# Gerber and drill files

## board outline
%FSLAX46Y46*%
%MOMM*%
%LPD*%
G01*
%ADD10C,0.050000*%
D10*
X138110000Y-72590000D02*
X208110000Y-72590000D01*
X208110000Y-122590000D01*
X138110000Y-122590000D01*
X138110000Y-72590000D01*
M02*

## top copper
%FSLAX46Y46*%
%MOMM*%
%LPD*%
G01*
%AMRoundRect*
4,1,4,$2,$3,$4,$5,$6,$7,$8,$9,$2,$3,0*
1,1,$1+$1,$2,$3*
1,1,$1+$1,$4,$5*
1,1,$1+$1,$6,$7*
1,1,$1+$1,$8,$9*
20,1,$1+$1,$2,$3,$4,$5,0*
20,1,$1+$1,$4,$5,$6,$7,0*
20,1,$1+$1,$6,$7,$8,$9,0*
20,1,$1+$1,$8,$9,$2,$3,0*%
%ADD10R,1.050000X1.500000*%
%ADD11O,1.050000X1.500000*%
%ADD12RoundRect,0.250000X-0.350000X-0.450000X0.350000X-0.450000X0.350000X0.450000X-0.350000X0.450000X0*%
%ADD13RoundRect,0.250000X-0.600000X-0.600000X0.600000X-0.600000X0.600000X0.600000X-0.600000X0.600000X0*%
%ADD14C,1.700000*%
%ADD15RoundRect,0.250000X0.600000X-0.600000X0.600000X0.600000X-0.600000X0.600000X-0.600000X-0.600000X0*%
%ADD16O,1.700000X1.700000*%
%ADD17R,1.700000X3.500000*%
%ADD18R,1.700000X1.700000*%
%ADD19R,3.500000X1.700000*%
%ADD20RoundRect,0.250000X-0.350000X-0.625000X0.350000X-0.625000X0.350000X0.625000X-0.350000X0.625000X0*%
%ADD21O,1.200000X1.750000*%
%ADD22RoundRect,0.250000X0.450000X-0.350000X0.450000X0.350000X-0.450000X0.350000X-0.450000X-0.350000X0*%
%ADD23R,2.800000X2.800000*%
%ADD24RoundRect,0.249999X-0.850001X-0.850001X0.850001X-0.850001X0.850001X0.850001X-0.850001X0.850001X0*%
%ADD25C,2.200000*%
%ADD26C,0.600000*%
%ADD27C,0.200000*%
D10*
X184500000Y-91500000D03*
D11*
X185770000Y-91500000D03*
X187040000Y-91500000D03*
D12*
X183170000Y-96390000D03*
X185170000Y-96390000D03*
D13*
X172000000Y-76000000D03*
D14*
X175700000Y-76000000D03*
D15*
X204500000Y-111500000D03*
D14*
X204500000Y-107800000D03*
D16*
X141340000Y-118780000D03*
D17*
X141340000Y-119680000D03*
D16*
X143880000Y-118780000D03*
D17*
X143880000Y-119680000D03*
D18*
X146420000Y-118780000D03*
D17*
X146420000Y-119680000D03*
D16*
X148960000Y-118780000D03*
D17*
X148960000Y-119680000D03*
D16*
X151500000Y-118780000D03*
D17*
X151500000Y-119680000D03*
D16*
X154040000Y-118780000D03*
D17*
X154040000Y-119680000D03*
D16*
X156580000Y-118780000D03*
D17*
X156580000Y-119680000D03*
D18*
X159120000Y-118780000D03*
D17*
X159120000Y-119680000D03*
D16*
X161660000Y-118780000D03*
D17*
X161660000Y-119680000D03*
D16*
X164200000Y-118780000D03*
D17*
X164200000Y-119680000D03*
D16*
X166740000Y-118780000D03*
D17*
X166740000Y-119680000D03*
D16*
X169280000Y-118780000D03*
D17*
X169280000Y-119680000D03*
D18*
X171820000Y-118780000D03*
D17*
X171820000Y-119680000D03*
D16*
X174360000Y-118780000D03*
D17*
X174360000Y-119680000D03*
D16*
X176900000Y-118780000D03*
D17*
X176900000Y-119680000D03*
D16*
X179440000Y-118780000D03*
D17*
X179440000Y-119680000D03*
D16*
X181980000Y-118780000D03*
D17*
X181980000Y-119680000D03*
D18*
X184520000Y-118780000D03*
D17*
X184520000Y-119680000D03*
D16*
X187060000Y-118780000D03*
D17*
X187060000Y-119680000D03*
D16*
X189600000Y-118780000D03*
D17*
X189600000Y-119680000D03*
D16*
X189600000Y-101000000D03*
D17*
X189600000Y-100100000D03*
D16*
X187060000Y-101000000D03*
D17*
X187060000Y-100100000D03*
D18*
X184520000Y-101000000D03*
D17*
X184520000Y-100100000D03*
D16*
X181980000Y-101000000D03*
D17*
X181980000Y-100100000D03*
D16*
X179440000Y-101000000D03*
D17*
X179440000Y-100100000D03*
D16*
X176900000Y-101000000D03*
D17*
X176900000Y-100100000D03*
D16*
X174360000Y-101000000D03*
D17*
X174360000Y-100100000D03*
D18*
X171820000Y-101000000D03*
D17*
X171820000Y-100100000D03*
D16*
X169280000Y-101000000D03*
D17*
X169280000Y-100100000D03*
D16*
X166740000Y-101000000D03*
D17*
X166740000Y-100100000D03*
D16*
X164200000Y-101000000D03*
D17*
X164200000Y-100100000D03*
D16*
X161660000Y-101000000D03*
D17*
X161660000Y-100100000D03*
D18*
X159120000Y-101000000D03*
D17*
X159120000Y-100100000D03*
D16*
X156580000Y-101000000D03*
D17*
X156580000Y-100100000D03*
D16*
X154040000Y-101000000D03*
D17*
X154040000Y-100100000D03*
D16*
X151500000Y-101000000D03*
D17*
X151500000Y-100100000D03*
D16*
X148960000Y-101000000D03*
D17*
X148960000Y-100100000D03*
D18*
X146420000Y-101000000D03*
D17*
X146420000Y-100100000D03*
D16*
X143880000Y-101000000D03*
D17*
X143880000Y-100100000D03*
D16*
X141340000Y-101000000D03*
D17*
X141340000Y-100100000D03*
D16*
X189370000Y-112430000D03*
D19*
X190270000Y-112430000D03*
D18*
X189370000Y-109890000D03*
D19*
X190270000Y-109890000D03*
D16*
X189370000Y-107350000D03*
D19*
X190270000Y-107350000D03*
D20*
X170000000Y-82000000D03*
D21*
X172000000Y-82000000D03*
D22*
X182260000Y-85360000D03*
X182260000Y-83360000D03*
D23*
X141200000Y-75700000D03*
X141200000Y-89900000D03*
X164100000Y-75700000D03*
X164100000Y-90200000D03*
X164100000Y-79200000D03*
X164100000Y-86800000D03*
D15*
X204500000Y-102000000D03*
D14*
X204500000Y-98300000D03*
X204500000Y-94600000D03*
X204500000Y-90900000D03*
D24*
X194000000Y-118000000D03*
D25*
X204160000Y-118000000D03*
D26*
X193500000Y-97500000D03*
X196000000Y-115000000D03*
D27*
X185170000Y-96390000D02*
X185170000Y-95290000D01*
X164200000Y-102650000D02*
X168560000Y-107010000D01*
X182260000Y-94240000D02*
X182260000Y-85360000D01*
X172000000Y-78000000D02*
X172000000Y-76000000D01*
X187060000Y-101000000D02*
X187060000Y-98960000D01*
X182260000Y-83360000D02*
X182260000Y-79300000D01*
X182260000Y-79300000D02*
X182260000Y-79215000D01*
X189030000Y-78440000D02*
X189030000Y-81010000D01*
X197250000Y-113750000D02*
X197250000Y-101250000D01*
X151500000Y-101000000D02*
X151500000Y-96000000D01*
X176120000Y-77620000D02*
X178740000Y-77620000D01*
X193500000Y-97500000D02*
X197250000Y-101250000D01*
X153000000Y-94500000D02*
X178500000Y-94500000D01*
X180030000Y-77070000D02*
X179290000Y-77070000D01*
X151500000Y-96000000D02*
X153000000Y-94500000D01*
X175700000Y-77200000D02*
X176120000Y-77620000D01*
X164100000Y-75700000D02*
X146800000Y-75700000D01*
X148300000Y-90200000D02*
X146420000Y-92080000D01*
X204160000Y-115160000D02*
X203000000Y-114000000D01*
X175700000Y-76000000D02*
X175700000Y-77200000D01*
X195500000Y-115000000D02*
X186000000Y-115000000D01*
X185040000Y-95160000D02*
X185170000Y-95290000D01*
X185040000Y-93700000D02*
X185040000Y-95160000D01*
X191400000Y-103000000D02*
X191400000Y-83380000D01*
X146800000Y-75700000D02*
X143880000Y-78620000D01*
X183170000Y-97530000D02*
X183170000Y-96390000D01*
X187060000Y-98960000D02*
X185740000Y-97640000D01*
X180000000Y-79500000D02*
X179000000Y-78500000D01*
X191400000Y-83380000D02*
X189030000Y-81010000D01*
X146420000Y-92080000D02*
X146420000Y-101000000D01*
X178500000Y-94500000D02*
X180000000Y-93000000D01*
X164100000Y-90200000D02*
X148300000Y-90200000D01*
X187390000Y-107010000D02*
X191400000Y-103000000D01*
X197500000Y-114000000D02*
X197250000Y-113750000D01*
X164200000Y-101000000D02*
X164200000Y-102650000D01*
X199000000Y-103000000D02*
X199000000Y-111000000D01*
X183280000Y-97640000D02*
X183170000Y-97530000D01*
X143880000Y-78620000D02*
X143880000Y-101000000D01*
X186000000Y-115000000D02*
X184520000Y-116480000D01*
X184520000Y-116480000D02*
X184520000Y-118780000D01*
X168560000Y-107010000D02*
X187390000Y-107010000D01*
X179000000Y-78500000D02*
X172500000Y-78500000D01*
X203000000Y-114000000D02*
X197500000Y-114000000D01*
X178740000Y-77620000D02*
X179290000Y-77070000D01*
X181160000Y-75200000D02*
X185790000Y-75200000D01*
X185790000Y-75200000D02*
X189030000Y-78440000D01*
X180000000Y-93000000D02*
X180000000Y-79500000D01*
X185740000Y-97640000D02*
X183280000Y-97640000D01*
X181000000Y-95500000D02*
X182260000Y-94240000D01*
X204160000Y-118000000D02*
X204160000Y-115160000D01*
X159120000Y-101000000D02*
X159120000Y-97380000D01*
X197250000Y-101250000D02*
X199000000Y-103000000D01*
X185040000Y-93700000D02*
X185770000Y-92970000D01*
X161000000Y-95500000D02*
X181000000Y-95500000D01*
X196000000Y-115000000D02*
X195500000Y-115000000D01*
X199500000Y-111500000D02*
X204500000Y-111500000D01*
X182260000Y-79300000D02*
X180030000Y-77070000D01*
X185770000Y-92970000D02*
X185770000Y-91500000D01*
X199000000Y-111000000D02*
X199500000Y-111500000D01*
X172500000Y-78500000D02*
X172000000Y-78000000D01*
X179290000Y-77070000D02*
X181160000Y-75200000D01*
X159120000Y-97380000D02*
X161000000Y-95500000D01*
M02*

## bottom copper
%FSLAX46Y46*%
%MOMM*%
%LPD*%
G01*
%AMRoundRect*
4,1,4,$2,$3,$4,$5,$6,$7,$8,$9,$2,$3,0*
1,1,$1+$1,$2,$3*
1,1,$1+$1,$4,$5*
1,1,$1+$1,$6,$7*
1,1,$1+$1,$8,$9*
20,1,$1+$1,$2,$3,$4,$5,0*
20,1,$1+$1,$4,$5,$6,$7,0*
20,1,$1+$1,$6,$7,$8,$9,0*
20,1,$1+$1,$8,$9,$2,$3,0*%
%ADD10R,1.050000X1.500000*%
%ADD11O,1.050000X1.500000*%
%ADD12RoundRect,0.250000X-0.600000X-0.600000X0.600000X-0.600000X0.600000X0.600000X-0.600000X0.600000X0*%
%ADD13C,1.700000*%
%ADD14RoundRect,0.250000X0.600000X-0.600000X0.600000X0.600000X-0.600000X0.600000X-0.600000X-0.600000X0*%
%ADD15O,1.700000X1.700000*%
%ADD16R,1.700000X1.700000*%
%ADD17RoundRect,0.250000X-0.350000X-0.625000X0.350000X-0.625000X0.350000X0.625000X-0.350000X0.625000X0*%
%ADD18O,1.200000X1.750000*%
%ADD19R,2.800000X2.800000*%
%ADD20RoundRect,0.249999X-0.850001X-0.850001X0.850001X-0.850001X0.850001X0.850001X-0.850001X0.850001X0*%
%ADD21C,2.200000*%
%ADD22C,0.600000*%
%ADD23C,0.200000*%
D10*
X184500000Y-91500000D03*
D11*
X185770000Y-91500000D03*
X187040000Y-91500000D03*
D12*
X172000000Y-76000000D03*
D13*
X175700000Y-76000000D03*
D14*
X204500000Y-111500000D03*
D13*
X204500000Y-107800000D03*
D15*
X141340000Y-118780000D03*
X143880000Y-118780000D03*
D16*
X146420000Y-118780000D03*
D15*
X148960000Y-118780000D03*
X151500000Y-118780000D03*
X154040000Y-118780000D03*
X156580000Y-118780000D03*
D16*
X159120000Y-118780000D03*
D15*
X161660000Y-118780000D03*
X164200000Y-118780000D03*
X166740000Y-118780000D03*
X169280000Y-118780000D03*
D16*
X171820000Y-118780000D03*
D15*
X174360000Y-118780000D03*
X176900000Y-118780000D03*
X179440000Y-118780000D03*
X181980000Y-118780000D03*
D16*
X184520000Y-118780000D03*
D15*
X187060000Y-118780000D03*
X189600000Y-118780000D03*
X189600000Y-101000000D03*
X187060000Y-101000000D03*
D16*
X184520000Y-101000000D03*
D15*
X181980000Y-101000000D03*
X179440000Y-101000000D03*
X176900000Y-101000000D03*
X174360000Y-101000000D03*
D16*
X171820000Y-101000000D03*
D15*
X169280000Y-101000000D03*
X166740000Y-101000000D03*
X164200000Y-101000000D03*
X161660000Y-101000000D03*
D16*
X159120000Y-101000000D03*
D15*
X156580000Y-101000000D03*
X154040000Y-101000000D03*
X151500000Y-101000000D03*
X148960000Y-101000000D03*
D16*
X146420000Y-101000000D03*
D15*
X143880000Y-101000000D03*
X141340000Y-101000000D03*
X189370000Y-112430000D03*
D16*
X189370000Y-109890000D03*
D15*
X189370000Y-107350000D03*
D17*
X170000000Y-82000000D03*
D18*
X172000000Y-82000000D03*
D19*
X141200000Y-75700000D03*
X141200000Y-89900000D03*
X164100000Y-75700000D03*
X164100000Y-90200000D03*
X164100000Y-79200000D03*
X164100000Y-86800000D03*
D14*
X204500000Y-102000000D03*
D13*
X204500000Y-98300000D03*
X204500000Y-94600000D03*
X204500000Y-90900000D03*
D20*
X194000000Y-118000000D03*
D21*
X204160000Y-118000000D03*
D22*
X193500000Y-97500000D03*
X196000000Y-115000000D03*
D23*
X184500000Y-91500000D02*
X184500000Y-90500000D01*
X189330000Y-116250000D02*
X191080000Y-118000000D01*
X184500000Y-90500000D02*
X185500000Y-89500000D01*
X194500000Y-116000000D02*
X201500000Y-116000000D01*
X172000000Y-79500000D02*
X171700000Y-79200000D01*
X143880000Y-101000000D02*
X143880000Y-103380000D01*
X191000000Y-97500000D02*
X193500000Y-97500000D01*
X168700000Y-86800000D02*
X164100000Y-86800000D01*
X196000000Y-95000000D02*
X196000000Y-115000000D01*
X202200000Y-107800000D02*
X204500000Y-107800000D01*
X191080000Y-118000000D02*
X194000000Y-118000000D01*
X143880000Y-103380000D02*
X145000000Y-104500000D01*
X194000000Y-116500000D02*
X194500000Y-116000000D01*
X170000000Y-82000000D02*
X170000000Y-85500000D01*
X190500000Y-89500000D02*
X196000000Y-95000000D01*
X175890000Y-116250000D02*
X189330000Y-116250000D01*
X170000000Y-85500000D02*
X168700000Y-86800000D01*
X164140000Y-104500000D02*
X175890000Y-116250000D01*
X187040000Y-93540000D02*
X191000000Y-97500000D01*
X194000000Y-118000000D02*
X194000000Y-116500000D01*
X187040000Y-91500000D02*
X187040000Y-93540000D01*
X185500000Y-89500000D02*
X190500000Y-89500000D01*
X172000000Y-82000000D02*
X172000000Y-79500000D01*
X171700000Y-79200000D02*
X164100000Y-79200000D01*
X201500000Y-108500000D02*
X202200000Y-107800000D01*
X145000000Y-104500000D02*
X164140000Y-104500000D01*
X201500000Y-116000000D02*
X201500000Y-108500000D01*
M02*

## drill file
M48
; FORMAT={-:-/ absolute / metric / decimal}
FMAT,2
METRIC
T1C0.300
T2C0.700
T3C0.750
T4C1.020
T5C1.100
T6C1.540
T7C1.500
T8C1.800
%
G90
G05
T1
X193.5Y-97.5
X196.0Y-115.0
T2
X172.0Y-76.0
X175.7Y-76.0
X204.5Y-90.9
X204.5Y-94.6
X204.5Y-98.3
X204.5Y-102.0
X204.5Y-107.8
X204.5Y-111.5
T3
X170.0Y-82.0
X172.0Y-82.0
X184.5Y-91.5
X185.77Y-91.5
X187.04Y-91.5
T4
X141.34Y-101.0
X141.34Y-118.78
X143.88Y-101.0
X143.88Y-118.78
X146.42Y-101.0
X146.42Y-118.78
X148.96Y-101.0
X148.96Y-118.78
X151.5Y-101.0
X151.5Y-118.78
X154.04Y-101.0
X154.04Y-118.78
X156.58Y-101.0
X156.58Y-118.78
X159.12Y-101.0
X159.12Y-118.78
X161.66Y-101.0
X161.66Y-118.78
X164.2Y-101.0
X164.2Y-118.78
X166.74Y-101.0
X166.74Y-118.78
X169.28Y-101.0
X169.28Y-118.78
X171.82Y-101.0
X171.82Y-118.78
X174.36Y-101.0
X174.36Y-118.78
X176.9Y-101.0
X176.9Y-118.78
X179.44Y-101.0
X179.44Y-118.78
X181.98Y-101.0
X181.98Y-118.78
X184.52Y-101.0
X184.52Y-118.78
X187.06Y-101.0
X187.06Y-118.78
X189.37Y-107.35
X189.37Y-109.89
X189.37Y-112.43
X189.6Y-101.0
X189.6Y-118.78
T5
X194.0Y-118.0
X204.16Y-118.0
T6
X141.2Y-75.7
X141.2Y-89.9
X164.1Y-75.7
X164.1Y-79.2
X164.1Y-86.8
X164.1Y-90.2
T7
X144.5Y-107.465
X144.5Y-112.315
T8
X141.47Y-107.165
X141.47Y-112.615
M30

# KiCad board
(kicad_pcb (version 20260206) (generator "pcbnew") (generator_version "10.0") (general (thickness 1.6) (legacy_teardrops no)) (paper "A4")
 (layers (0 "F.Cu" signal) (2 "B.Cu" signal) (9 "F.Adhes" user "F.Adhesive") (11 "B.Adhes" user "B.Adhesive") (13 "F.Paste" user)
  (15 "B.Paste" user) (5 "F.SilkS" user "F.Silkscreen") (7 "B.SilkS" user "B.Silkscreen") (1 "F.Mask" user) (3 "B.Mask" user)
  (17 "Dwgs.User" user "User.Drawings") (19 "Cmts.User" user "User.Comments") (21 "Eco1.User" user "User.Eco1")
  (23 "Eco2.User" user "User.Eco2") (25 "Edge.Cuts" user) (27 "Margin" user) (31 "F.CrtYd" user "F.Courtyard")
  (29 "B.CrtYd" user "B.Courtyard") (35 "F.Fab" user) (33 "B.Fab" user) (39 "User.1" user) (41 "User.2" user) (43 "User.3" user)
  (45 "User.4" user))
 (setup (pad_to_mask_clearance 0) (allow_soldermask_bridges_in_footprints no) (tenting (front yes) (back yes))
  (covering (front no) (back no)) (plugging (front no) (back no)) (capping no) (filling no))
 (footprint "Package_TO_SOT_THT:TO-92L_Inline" (layer "F.Cu") (at 184.5 91.5)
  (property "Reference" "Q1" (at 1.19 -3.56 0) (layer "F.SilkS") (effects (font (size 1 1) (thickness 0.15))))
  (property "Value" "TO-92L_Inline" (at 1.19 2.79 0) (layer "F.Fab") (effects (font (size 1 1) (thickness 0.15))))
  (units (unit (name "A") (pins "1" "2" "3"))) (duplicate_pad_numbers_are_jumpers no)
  (pad "1" thru_hole rect (at 0 0) (size 1.05 1.5) (drill 0.75) (layers "*.Cu" "*.Mask") (remove_unused_layers no))
  (pad "2" thru_hole oval (at 1.27 0) (size 1.05 1.5) (drill 0.75) (layers "*.Cu" "*.Mask") (remove_unused_layers no))
  (pad "3" thru_hole oval (at 2.54 0) (size 1.05 1.5) (drill 0.75) (layers "*.Cu" "*.Mask") (remove_unused_layers no)))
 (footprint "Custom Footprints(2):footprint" (layer "F.Cu") (at 202 78.55)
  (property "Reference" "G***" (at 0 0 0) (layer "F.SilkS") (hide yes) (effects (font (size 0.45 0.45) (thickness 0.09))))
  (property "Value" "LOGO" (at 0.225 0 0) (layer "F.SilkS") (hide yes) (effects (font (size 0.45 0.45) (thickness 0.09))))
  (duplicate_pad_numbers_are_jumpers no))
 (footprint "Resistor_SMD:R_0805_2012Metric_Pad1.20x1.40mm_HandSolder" (layer "F.Cu") (at 184.17 96.39)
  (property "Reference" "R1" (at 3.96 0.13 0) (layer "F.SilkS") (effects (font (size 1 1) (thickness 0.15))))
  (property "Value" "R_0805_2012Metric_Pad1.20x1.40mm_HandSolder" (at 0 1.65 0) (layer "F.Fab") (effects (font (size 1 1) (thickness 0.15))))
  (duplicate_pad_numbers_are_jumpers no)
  (pad "1" smd roundrect (at -1 0) (size 1.2 1.4) (layers "F.Cu" "F.Mask" "F.Paste") (roundrect_rratio 0.208333))
  (pad "2" smd roundrect (at 1 0) (size 1.2 1.4) (layers "F.Cu" "F.Mask" "F.Paste") (roundrect_rratio 0.208333)))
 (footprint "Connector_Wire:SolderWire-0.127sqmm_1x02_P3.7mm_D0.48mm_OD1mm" (layer "F.Cu") (at 172 76)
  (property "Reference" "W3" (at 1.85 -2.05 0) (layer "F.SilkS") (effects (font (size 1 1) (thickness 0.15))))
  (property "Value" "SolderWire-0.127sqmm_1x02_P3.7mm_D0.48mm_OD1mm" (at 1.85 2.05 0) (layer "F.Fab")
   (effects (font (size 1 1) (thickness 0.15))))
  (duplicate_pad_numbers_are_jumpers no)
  (pad "1" thru_hole roundrect (at 0 0) (size 1.7 1.7) (drill 0.7) (layers "*.Cu" "*.Mask") (remove_unused_layers no)
   (roundrect_rratio 0.147059))
  (pad "2" thru_hole circle (at 3.7 0) (size 1.7 1.7) (drill 0.7) (layers "*.Cu" "*.Mask") (remove_unused_layers no)))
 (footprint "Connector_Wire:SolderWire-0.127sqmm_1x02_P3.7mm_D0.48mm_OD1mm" (layer "F.Cu") (at 204.5 111.5 90)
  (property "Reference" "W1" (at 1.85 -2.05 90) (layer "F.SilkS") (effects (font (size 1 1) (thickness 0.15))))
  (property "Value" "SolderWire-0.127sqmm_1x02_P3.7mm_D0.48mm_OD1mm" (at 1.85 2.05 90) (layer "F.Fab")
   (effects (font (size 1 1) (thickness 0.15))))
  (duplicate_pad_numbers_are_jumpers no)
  (pad "1" thru_hole roundrect (at 0 0 90) (size 1.7 1.7) (drill 0.7) (layers "*.Cu" "*.Mask") (remove_unused_layers no)
   (roundrect_rratio 0.147059))
  (pad "2" thru_hole circle (at 3.7 0 90) (size 1.7 1.7) (drill 0.7) (layers "*.Cu" "*.Mask") (remove_unused_layers no)))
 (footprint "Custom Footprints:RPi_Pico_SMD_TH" (layer "F.Cu") (at 165.47 109.89 90)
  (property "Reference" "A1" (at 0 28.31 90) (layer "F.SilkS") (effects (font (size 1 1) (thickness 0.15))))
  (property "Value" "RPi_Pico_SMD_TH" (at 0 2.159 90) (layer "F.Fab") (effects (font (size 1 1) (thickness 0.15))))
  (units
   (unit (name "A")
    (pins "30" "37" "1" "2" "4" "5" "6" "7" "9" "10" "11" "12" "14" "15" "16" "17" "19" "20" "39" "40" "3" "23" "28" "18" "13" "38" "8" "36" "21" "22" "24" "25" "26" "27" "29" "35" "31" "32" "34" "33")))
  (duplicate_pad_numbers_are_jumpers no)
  (pad "" np_thru_hole oval (at -2.725 -24 90) (size 1.8 1.8) (drill 1.8) (layers "*.Cu" "*.Mask"))
  (pad "" np_thru_hole oval (at -2.425 -20.97 90) (size 1.5 1.5) (drill 1.5) (layers "*.Cu" "*.Mask"))
  (pad "" np_thru_hole oval (at 2.425 -20.97 90) (size 1.5 1.5) (drill 1.5) (layers "*.Cu" "*.Mask"))
  (pad "" np_thru_hole oval (at 2.725 -24 90) (size 1.8 1.8) (drill 1.8) (layers "*.Cu" "*.Mask"))
  (pad "1" thru_hole oval (at -8.89 -24.13 90) (size 1.7 1.7) (drill 1.02) (layers "*.Cu" "*.Mask") (remove_unused_layers no))
  (pad "1" smd rect (at -8.89 -24.13 90) (size 3.5 1.7) (drill (offset -0.9 0)) (layers "F.Cu" "F.Mask"))
  (pad "2" thru_hole oval (at -8.89 -21.59 90) (size 1.7 1.7) (drill 1.02) (layers "*.Cu" "*.Mask") (remove_unused_layers no))
  (pad "2" smd rect (at -8.89 -21.59 90) (size 3.5 1.7) (drill (offset -0.9 0)) (layers "F.Cu" "F.Mask"))
  (pad "3" thru_hole rect (at -8.89 -19.05 90) (size 1.7 1.7) (drill 1.02) (layers "*.Cu" "*.Mask") (remove_unused_layers no))
  (pad "3" smd rect (at -8.89 -19.05 90) (size 3.5 1.7) (drill (offset -0.9 0)) (layers "F.Cu" "F.Mask"))
  (pad "4" thru_hole oval (at -8.89 -16.51 90) (size 1.7 1.7) (drill 1.02) (layers "*.Cu" "*.Mask") (remove_unused_layers no))
  (pad "4" smd rect (at -8.89 -16.51 90) (size 3.5 1.7) (drill (offset -0.9 0)) (layers "F.Cu" "F.Mask"))
  (pad "5" thru_hole oval (at -8.89 -13.97 90) (size 1.7 1.7) (drill 1.02) (layers "*.Cu" "*.Mask") (remove_unused_layers no))
  (pad "5" smd rect (at -8.89 -13.97 90) (size 3.5 1.7) (drill (offset -0.9 0)) (layers "F.Cu" "F.Mask"))
  (pad "6" thru_hole oval (at -8.89 -11.43 90) (size 1.7 1.7) (drill 1.02) (layers "*.Cu" "*.Mask") (remove_unused_layers no))
  (pad "6" smd rect (at -8.89 -11.43 90) (size 3.5 1.7) (drill (offset -0.9 0)) (layers "F.Cu" "F.Mask"))
  (pad "7" thru_hole oval (at -8.89 -8.89 90) (size 1.7 1.7) (drill 1.02) (layers "*.Cu" "*.Mask") (remove_unused_layers no))
  (pad "7" smd rect (at -8.89 -8.89 90) (size 3.5 1.7) (drill (offset -0.9 0)) (layers "F.Cu" "F.Mask"))
  (pad "8" thru_hole rect (at -8.89 -6.35 90) (size 1.7 1.7) (drill 1.02) (layers "*.Cu" "*.Mask") (remove_unused_layers no))
  (pad "8" smd rect (at -8.89 -6.35 90) (size 3.5 1.7) (drill (offset -0.9 0)) (layers "F.Cu" "F.Mask"))
  (pad "9" thru_hole oval (at -8.89 -3.81 90) (size 1.7 1.7) (drill 1.02) (layers "*.Cu" "*.Mask") (remove_unused_layers no))
  (pad "9" smd rect (at -8.89 -3.81 90) (size 3.5 1.7) (drill (offset -0.9 0)) (layers "F.Cu" "F.Mask"))
  (pad "10" thru_hole oval (at -8.89 -1.27 90) (size 1.7 1.7) (drill 1.02) (layers "*.Cu" "*.Mask") (remove_unused_layers no))
  (pad "10" smd rect (at -8.89 -1.27 90) (size 3.5 1.7) (drill (offset -0.9 0)) (layers "F.Cu" "F.Mask"))
  (pad "11" thru_hole oval (at -8.89 1.27 90) (size 1.7 1.7) (drill 1.02) (layers "*.Cu" "*.Mask") (remove_unused_layers no))
  (pad "11" smd rect (at -8.89 1.27 90) (size 3.5 1.7) (drill (offset -0.9 0)) (layers "F.Cu" "F.Mask"))
  (pad "12" thru_hole oval (at -8.89 3.81 90) (size 1.7 1.7) (drill 1.02) (layers "*.Cu" "*.Mask") (remove_unused_layers no))
  (pad "12" smd rect (at -8.89 3.81 90) (size 3.5 1.7) (drill (offset -0.9 0)) (layers "F.Cu" "F.Mask"))
  (pad "13" thru_hole rect (at -8.89 6.35 90) (size 1.7 1.7) (drill 1.02) (layers "*.Cu" "*.Mask") (remove_unused_layers no))
  (pad "13" smd rect (at -8.89 6.35 90) (size 3.5 1.7) (drill (offset -0.9 0)) (layers "F.Cu" "F.Mask"))
  (pad "14" thru_hole oval (at -8.89 8.89 90) (size 1.7 1.7) (drill 1.02) (layers "*.Cu" "*.Mask") (remove_unused_layers no))
  (pad "14" smd rect (at -8.89 8.89 90) (size 3.5 1.7) (drill (offset -0.9 0)) (layers "F.Cu" "F.Mask"))
  (pad "15" thru_hole oval (at -8.89 11.43 90) (size 1.7 1.7) (drill 1.02) (layers "*.Cu" "*.Mask") (remove_unused_layers no))
  (pad "15" smd rect (at -8.89 11.43 90) (size 3.5 1.7) (drill (offset -0.9 0)) (layers "F.Cu" "F.Mask"))
  (pad "16" thru_hole oval (at -8.89 13.97 90) (size 1.7 1.7) (drill 1.02) (layers "*.Cu" "*.Mask") (remove_unused_layers no))
  (pad "16" smd rect (at -8.89 13.97 90) (size 3.5 1.7) (drill (offset -0.9 0)) (layers "F.Cu" "F.Mask"))
  (pad "17" thru_hole oval (at -8.89 16.51 90) (size 1.7 1.7) (drill 1.02) (layers "*.Cu" "*.Mask") (remove_unused_layers no))
  (pad "17" smd rect (at -8.89 16.51 90) (size 3.5 1.7) (drill (offset -0.9 0)) (layers "F.Cu" "F.Mask"))
  (pad "18" thru_hole rect (at -8.89 19.05 90) (size 1.7 1.7) (drill 1.02) (layers "*.Cu" "*.Mask") (remove_unused_layers no))
  (pad "18" smd rect (at -8.89 19.05 90) (size 3.5 1.7) (drill (offset -0.9 0)) (layers "F.Cu" "F.Mask"))
  (pad "19" thru_hole oval (at -8.89 21.59 90) (size 1.7 1.7) (drill 1.02) (layers "*.Cu" "*.Mask") (remove_unused_layers no))
  (pad "19" smd rect (at -8.89 21.59 90) (size 3.5 1.7) (drill (offset -0.9 0)) (layers "F.Cu" "F.Mask"))
  (pad "20" thru_hole oval (at -8.89 24.13 90) (size 1.7 1.7) (drill 1.02) (layers "*.Cu" "*.Mask") (remove_unused_layers no))
  (pad "20" smd rect (at -8.89 24.13 90) (size 3.5 1.7) (drill (offset -0.9 0)) (layers "F.Cu" "F.Mask"))
  (pad "21" thru_hole oval (at 8.89 24.13 90) (size 1.7 1.7) (drill 1.02) (layers "*.Cu" "*.Mask") (remove_unused_layers no))
  (pad "21" smd rect (at 8.89 24.13 90) (size 3.5 1.7) (drill (offset 0.9 0)) (layers "F.Cu" "F.Mask"))
  (pad "22" thru_hole oval (at 8.89 21.59 90) (size 1.7 1.7) (drill 1.02) (layers "*.Cu" "*.Mask") (remove_unused_layers no))
  (pad "22" smd rect (at 8.89 21.59 90) (size 3.5 1.7) (drill (offset 0.9 0)) (layers "F.Cu" "F.Mask"))
  (pad "23" thru_hole rect (at 8.89 19.05 90) (size 1.7 1.7) (drill 1.02) (layers "*.Cu" "*.Mask") (remove_unused_layers no))
  (pad "23" smd rect (at 8.89 19.05 90) (size 3.5 1.7) (drill (offset 0.9 0)) (layers "F.Cu" "F.Mask"))
  (pad "24" thru_hole oval (at 8.89 16.51 90) (size 1.7 1.7) (drill 1.02) (layers "*.Cu" "*.Mask") (remove_unused_layers no))
  (pad "24" smd rect (at 8.89 16.51 90) (size 3.5 1.7) (drill (offset 0.9 0)) (layers "F.Cu" "F.Mask"))
  (pad "25" thru_hole oval (at 8.89 13.97 90) (size 1.7 1.7) (drill 1.02) (layers "*.Cu" "*.Mask") (remove_unused_layers no))
  (pad "25" smd rect (at 8.89 13.97 90) (size 3.5 1.7) (drill (offset 0.9 0)) (layers "F.Cu" "F.Mask"))
  (pad "26" thru_hole oval (at 8.89 11.43 90) (size 1.7 1.7) (drill 1.02) (layers "*.Cu" "*.Mask") (remove_unused_layers no))
  (pad "26" smd rect (at 8.89 11.43 90) (size 3.5 1.7) (drill (offset 0.9 0)) (layers "F.Cu" "F.Mask"))
  (pad "27" thru_hole oval (at 8.89 8.89 90) (size 1.7 1.7) (drill 1.02) (layers "*.Cu" "*.Mask") (remove_unused_layers no))
  (pad "27" smd rect (at 8.89 8.89 90) (size 3.5 1.7) (drill (offset 0.9 0)) (layers "F.Cu" "F.Mask"))
  (pad "28" thru_hole rect (at 8.89 6.35 90) (size 1.7 1.7) (drill 1.02) (layers "*.Cu" "*.Mask") (remove_unused_layers no))
  (pad "28" smd rect (at 8.89 6.35 90) (size 3.5 1.7) (drill (offset 0.9 0)) (layers "F.Cu" "F.Mask"))
  (pad "29" thru_hole oval (at 8.89 3.81 90) (size 1.7 1.7) (drill 1.02) (layers "*.Cu" "*.Mask") (remove_unused_layers no))
  (pad "29" smd rect (at 8.89 3.81 90) (size 3.5 1.7) (drill (offset 0.9 0)) (layers "F.Cu" "F.Mask"))
  (pad "30" thru_hole oval (at 8.89 1.27 90) (size 1.7 1.7) (drill 1.02) (layers "*.Cu" "*.Mask") (remove_unused_layers no))
  (pad "30" smd rect (at 8.89 1.27 90) (size 3.5 1.7) (drill (offset 0.9 0)) (layers "F.Cu" "F.Mask"))
  (pad "31" thru_hole oval (at 8.89 -1.27 90) (size 1.7 1.7) (drill 1.02) (layers "*.Cu" "*.Mask") (remove_unused_layers no))
  (pad "31" smd rect (at 8.89 -1.27 90) (size 3.5 1.7) (drill (offset 0.9 0)) (layers "F.Cu" "F.Mask"))
  (pad "32" thru_hole oval (at 8.89 -3.81 90) (size 1.7 1.7) (drill 1.02) (layers "*.Cu" "*.Mask") (remove_unused_layers no))
  (pad "32" smd rect (at 8.89 -3.81 90) (size 3.5 1.7) (drill (offset 0.9 0)) (layers "F.Cu" "F.Mask"))
  (pad "33" thru_hole rect (at 8.89 -6.35 90) (size 1.7 1.7) (drill 1.02) (layers "*.Cu" "*.Mask") (remove_unused_layers no))
  (pad "33" smd rect (at 8.89 -6.35 90) (size 3.5 1.7) (drill (offset 0.9 0)) (layers "F.Cu" "F.Mask"))
  (pad "34" thru_hole oval (at 8.89 -8.89 90) (size 1.7 1.7) (drill 1.02) (layers "*.Cu" "*.Mask") (remove_unused_layers no))
  (pad "34" smd rect (at 8.89 -8.89 90) (size 3.5 1.7) (drill (offset 0.9 0)) (layers "F.Cu" "F.Mask"))
  (pad "35" thru_hole oval (at 8.89 -11.43 90) (size 1.7 1.7) (drill 1.02) (layers "*.Cu" "*.Mask") (remove_unused_layers no))
  (pad "35" smd rect (at 8.89 -11.43 90) (size 3.5 1.7) (drill (offset 0.9 0)) (layers "F.Cu" "F.Mask"))
  (pad "36" thru_hole oval (at 8.89 -13.97 90) (size 1.7 1.7) (drill 1.02) (layers "*.Cu" "*.Mask") (remove_unused_layers no))
  (pad "36" smd rect (at 8.89 -13.97 90) (size 3.5 1.7) (drill (offset 0.9 0)) (layers "F.Cu" "F.Mask"))
  (pad "37" thru_hole oval (at 8.89 -16.51 90) (size 1.7 1.7) (drill 1.02) (layers "*.Cu" "*.Mask") (remove_unused_layers no))
  (pad "37" smd rect (at 8.89 -16.51 90) (size 3.5 1.7) (drill (offset 0.9 0)) (layers "F.Cu" "F.Mask"))
  (pad "38" thru_hole rect (at 8.89 -19.05 90) (size 1.7 1.7) (drill 1.02) (layers "*.Cu" "*.Mask") (remove_unused_layers no))
  (pad "38" smd rect (at 8.89 -19.05 90) (size 3.5 1.7) (drill (offset 0.9 0)) (layers "F.Cu" "F.Mask"))
  (pad "39" thru_hole oval (at 8.89 -21.59 90) (size 1.7 1.7) (drill 1.02) (layers "*.Cu" "*.Mask") (remove_unused_layers no))
  (pad "39" smd rect (at 8.89 -21.59 90) (size 3.5 1.7) (drill (offset 0.9 0)) (layers "F.Cu" "F.Mask"))
  (pad "40" thru_hole oval (at 8.89 -24.13 90) (size 1.7 1.7) (drill 1.02) (layers "*.Cu" "*.Mask") (remove_unused_layers no))
  (pad "40" smd rect (at 8.89 -24.13 90) (size 3.5 1.7) (drill (offset 0.9 0)) (layers "F.Cu" "F.Mask"))
  (pad "41" thru_hole oval (at -2.54 23.9 90) (size 1.7 1.7) (drill 1.02) (layers "*.Cu" "*.Mask") (remove_unused_layers no))
  (pad "41" smd rect (at -2.54 23.9 180) (size 3.5 1.7) (drill (offset -0.9 0)) (layers "F.Cu" "F.Mask"))
  (pad "42" thru_hole rect (at 0 23.9 90) (size 1.7 1.7) (drill 1.02) (layers "*.Cu" "*.Mask") (remove_unused_layers no))
  (pad "42" smd rect (at 0 23.9 180) (size 3.5 1.7) (drill (offset -0.9 0)) (layers "F.Cu" "F.Mask"))
  (pad "43" thru_hole oval (at 2.54 23.9 90) (size 1.7 1.7) (drill 1.02) (layers "*.Cu" "*.Mask") (remove_unused_layers no))
  (pad "43" smd rect (at 2.54 23.9 180) (size 3.5 1.7) (drill (offset -0.9 0)) (layers "F.Cu" "F.Mask")))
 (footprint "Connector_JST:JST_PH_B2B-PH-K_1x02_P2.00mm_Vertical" (layer "F.Cu") (at 170 82)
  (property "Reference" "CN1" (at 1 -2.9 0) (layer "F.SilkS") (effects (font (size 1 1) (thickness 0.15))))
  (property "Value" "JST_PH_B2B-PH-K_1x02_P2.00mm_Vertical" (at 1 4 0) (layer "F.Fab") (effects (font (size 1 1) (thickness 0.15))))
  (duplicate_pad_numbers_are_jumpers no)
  (pad "1" thru_hole roundrect (at 0 0) (size 1.2 1.75) (drill 0.75) (layers "*.Cu" "*.Mask") (remove_unused_layers no)
   (roundrect_rratio 0.208333))
  (pad "2" thru_hole oval (at 2 0) (size 1.2 1.75) (drill 0.75) (layers "*.Cu" "*.Mask") (remove_unused_layers no)))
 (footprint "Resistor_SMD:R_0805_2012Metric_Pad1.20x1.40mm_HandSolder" (layer "F.Cu") (at 182.26 84.36 90)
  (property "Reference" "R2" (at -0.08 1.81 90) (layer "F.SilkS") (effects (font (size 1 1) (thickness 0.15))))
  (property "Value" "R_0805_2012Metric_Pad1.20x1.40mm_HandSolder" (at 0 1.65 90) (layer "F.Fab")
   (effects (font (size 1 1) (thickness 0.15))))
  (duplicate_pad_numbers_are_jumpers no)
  (pad "1" smd roundrect (at -1 0 90) (size 1.2 1.4) (layers "F.Cu" "F.Mask" "F.Paste") (roundrect_rratio 0.208333))
  (pad "2" smd roundrect (at 1 0 90) (size 1.2 1.4) (layers "F.Cu" "F.Mask" "F.Paste") (roundrect_rratio 0.208333)))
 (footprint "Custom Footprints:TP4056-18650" (layer "F.Cu") (at 139.5 74)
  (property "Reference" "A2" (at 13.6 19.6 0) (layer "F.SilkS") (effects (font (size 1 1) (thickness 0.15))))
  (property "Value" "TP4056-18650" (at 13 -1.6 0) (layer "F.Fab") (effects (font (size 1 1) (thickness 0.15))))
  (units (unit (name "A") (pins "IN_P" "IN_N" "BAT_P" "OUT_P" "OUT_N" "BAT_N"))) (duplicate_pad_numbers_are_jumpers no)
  (pad "1" thru_hole rect (at 1.7 1.7) (size 2.8 2.8) (drill 1.54) (layers "*.Cu" "*.Mask") (remove_unused_layers no))
  (pad "2" thru_hole rect (at 1.7 15.9) (size 2.8 2.8) (drill 1.54) (layers "*.Cu" "*.Mask") (remove_unused_layers no))
  (pad "3" thru_hole rect (at 24.6 1.7) (size 2.8 2.8) (drill 1.54) (layers "*.Cu" "*.Mask") (remove_unused_layers no))
  (pad "4" thru_hole rect (at 24.6 16.2) (size 2.8 2.8) (drill 1.54) (layers "*.Cu" "*.Mask") (remove_unused_layers no))
  (pad "5" thru_hole rect (at 24.6 5.2) (size 2.8 2.8) (drill 1.54) (layers "*.Cu" "*.Mask") (remove_unused_layers no))
  (pad "6" thru_hole rect (at 24.6 12.8) (size 2.8 2.8) (drill 1.54) (layers "*.Cu" "*.Mask") (remove_unused_layers no)))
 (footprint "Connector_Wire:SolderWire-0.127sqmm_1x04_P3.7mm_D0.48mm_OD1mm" (layer "F.Cu") (at 204.5 102 90)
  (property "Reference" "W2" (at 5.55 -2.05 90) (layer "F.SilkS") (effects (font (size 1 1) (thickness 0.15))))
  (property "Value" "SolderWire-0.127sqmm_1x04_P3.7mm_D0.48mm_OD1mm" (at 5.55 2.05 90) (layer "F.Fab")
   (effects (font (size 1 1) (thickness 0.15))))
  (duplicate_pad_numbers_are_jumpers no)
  (pad "1" thru_hole roundrect (at 0 0 90) (size 1.7 1.7) (drill 0.7) (layers "*.Cu" "*.Mask") (remove_unused_layers no)
   (roundrect_rratio 0.147059))
  (pad "2" thru_hole circle (at 3.7 0 90) (size 1.7 1.7) (drill 0.7) (layers "*.Cu" "*.Mask") (remove_unused_layers no))
  (pad "3" thru_hole circle (at 7.4 0 90) (size 1.7 1.7) (drill 0.7) (layers "*.Cu" "*.Mask") (remove_unused_layers no))
  (pad "4" thru_hole circle (at 11.1 0 90) (size 1.7 1.7) (drill 0.7) (layers "*.Cu" "*.Mask") (remove_unused_layers no)))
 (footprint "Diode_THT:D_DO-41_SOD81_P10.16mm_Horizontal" (layer "F.Cu") (at 194 118)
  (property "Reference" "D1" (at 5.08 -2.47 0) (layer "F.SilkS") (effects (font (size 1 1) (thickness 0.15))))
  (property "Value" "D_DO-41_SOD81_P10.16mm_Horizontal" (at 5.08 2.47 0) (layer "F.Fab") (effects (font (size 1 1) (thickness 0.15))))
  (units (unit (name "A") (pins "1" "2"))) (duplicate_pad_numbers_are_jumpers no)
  (pad "1" thru_hole roundrect (at 0 0) (size 2.2 2.2) (drill 1.1) (layers "*.Cu" "*.Mask") (remove_unused_layers no)
   (roundrect_rratio 0.113636))
  (pad "2" thru_hole circle (at 10.16 0) (size 2.2 2.2) (drill 1.1) (layers "*.Cu" "*.Mask") (remove_unused_layers no)))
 (gr_rect (start 138.11 72.59) (end 208.11 122.59) (stroke (width 0.05) (type default)) (fill no) (layer "Edge.Cuts"))
 (segment (start 185.17 96.39) (end 185.17 95.29) (width 0.2) (layer "F.Cu") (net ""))
 (segment (start 164.2 102.65) (end 168.56 107.01) (width 0.2) (layer "F.Cu") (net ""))
 (segment (start 182.26 94.24) (end 182.26 85.36) (width 0.2) (layer "F.Cu") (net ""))
 (segment (start 172 78) (end 172 76) (width 0.2) (layer "F.Cu") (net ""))
 (segment (start 187.06 101) (end 187.06 98.96) (width 0.2) (layer "F.Cu") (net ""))
 (segment (start 182.26 83.36) (end 182.26 79.3) (width 0.2) (layer "F.Cu") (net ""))
 (segment (start 182.26 79.3) (end 182.26 79.215) (width 0.2) (layer "F.Cu") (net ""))
 (segment (start 189.03 78.44) (end 189.03 81.01) (width 0.2) (layer "F.Cu") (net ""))
 (segment (start 197.25 113.75) (end 197.25 101.25) (width 0.2) (layer "F.Cu") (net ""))
 (segment (start 151.5 101) (end 151.5 96) (width 0.2) (layer "F.Cu") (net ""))
 (segment (start 176.12 77.62) (end 178.74 77.62) (width 0.2) (layer "F.Cu") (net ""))
 (segment (start 193.5 97.5) (end 197.25 101.25) (width 0.2) (layer "F.Cu") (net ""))
 (segment (start 153 94.5) (end 178.5 94.5) (width 0.2) (layer "F.Cu") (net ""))
 (segment (start 180.03 77.07) (end 179.29 77.07) (width 0.2) (layer "F.Cu") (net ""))
 (segment (start 151.5 96) (end 153 94.5) (width 0.2) (layer "F.Cu") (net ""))
 (segment (start 175.7 77.2) (end 176.12 77.62) (width 0.2) (layer "F.Cu") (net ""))
 (segment (start 164.1 75.7) (end 146.8 75.7) (width 0.2) (layer "F.Cu") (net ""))
 (segment (start 148.3 90.2) (end 146.42 92.08) (width 0.2) (layer "F.Cu") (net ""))
 (segment (start 204.16 115.16) (end 203 114) (width 0.2) (layer "F.Cu") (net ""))
 (segment (start 175.7 76) (end 175.7 77.2) (width 0.2) (layer "F.Cu") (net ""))
 (segment (start 195.5 115) (end 186 115) (width 0.2) (layer "F.Cu") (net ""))
 (segment (start 185.04 95.16) (end 185.17 95.29) (width 0.2) (layer "F.Cu") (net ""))
 (segment (start 185.04 93.7) (end 185.04 95.16) (width 0.2) (layer "F.Cu") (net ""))
 (segment (start 191.4 103) (end 191.4 83.38) (width 0.2) (layer "F.Cu") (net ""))
 (segment (start 146.8 75.7) (end 143.88 78.62) (width 0.2) (layer "F.Cu") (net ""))
 (segment (start 183.17 97.53) (end 183.17 96.39) (width 0.2) (layer "F.Cu") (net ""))
 (segment (start 187.06 98.96) (end 185.74 97.64) (width 0.2) (layer "F.Cu") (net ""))
 (segment (start 180 79.5) (end 179 78.5) (width 0.2) (layer "F.Cu") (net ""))
 (segment (start 191.4 83.38) (end 189.03 81.01) (width 0.2) (layer "F.Cu") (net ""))
 (segment (start 146.42 92.08) (end 146.42 101) (width 0.2) (layer "F.Cu") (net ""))
 (segment (start 178.5 94.5) (end 180 93) (width 0.2) (layer "F.Cu") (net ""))
 (segment (start 164.1 90.2) (end 148.3 90.2) (width 0.2) (layer "F.Cu") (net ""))
 (segment (start 187.39 107.01) (end 191.4 103) (width 0.2) (layer "F.Cu") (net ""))
 (segment (start 197.5 114) (end 197.25 113.75) (width 0.2) (layer "F.Cu") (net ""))
 (segment (start 164.2 101) (end 164.2 102.65) (width 0.2) (layer "F.Cu") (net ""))
 (segment (start 199 103) (end 199 111) (width 0.2) (layer "F.Cu") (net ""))
 (segment (start 183.28 97.64) (end 183.17 97.53) (width 0.2) (layer "F.Cu") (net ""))
 (segment (start 143.88 78.62) (end 143.88 101) (width 0.2) (layer "F.Cu") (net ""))
 (segment (start 186 115) (end 184.52 116.48) (width 0.2) (layer "F.Cu") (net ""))
 (segment (start 184.52 116.48) (end 184.52 118.78) (width 0.2) (layer "F.Cu") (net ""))
 (segment (start 168.56 107.01) (end 187.39 107.01) (width 0.2) (layer "F.Cu") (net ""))
 (segment (start 179 78.5) (end 172.5 78.5) (width 0.2) (layer "F.Cu") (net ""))
 (segment (start 203 114) (end 197.5 114) (width 0.2) (layer "F.Cu") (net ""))
 (segment (start 178.74 77.62) (end 179.29 77.07) (width 0.2) (layer "F.Cu") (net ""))
 (segment (start 181.16 75.2) (end 185.79 75.2) (width 0.2) (layer "F.Cu") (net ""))
 (segment (start 185.79 75.2) (end 189.03 78.44) (width 0.2) (layer "F.Cu") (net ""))
 (segment (start 180 93) (end 180 79.5) (width 0.2) (layer "F.Cu") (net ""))
 (segment (start 185.74 97.64) (end 183.28 97.64) (width 0.2) (layer "F.Cu") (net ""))
 (segment (start 181 95.5) (end 182.26 94.24) (width 0.2) (layer "F.Cu") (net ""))
 (segment (start 204.16 118) (end 204.16 115.16) (width 0.2) (layer "F.Cu") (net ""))
 (segment (start 159.12 101) (end 159.12 97.38) (width 0.2) (layer "F.Cu") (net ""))
 (segment (start 197.25 101.25) (end 199 103) (width 0.2) (layer "F.Cu") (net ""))
 (segment (start 185.04 93.7) (end 185.77 92.97) (width 0.2) (layer "F.Cu") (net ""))
 (segment (start 161 95.5) (end 181 95.5) (width 0.2) (layer "F.Cu") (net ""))
 (segment (start 196 115) (end 195.5 115) (width 0.2) (layer "F.Cu") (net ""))
 (segment (start 199.5 111.5) (end 204.5 111.5) (width 0.2) (layer "F.Cu") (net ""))
 (segment (start 182.26 79.3) (end 180.03 77.07) (width 0.2) (layer "F.Cu") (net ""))
 (segment (start 185.77 92.97) (end 185.77 91.5) (width 0.2) (layer "F.Cu") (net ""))
 (segment (start 199 111) (end 199.5 111.5) (width 0.2) (layer "F.Cu") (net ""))
 (segment (start 172.5 78.5) (end 172 78) (width 0.2) (layer "F.Cu") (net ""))
 (segment (start 179.29 77.07) (end 181.16 75.2) (width 0.2) (layer "F.Cu") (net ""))
 (segment (start 159.12 97.38) (end 161 95.5) (width 0.2) (layer "F.Cu") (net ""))
 (via (at 193.5 97.5) (size 0.6) (drill 0.3) (layers "F.Cu" "B.Cu") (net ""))
 (via (at 196 115) (size 0.6) (drill 0.3) (layers "F.Cu" "B.Cu") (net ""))
 (segment (start 184.5 91.5) (end 184.5 90.5) (width 0.2) (layer "B.Cu") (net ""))
 (segment (start 189.33 116.25) (end 191.08 118) (width 0.2) (layer "B.Cu") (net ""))
 (segment (start 184.5 90.5) (end 185.5 89.5) (width 0.2) (layer "B.Cu") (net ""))
 (segment (start 194.5 116) (end 201.5 116) (width 0.2) (layer "B.Cu") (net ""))
 (segment (start 172 79.5) (end 171.7 79.2) (width 0.2) (layer "B.Cu") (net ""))
 (segment (start 143.88 101) (end 143.88 103.38) (width 0.2) (layer "B.Cu") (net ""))
 (segment (start 191 97.5) (end 193.5 97.5) (width 0.2) (layer "B.Cu") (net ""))
 (segment (start 168.7 86.8) (end 164.1 86.8) (width 0.2) (layer "B.Cu") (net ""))
 (segment (start 196 95) (end 196 115) (width 0.2) (layer "B.Cu") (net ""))
 (segment (start 202.2 107.8) (end 204.5 107.8) (width 0.2) (layer "B.Cu") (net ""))
 (segment (start 191.08 118) (end 194 118) (width 0.2) (layer "B.Cu") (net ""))
 (segment (start 143.88 103.38) (end 145 104.5) (width 0.2) (layer "B.Cu") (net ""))
 (segment (start 194 116.5) (end 194.5 116) (width 0.2) (layer "B.Cu") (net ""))
 (segment (start 170 82) (end 170 85.5) (width 0.2) (layer "B.Cu") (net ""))
 (segment (start 190.5 89.5) (end 196 95) (width 0.2) (layer "B.Cu") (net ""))
 (segment (start 175.89 116.25) (end 189.33 116.25) (width 0.2) (layer "B.Cu") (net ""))
 (segment (start 170 85.5) (end 168.7 86.8) (width 0.2) (layer "B.Cu") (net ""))
 (segment (start 164.14 104.5) (end 175.89 116.25) (width 0.2) (layer "B.Cu") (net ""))
 (segment (start 187.04 93.54) (end 191 97.5) (width 0.2) (layer "B.Cu") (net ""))
 (segment (start 194 118) (end 194 116.5) (width 0.2) (layer "B.Cu") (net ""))
 (segment (start 187.04 91.5) (end 187.04 93.54) (width 0.2) (layer "B.Cu") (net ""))
 (segment (start 185.5 89.5) (end 190.5 89.5) (width 0.2) (layer "B.Cu") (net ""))
 (segment (start 172 82) (end 172 79.5) (width 0.2) (layer "B.Cu") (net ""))
 (segment (start 171.7 79.2) (end 164.1 79.2) (width 0.2) (layer "B.Cu") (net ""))
 (segment (start 201.5 108.5) (end 202.2 107.8) (width 0.2) (layer "B.Cu") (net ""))
 (segment (start 145 104.5) (end 164.14 104.5) (width 0.2) (layer "B.Cu") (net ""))
 (segment (start 201.5 116) (end 201.5 108.5) (width 0.2) (layer "B.Cu") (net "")))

